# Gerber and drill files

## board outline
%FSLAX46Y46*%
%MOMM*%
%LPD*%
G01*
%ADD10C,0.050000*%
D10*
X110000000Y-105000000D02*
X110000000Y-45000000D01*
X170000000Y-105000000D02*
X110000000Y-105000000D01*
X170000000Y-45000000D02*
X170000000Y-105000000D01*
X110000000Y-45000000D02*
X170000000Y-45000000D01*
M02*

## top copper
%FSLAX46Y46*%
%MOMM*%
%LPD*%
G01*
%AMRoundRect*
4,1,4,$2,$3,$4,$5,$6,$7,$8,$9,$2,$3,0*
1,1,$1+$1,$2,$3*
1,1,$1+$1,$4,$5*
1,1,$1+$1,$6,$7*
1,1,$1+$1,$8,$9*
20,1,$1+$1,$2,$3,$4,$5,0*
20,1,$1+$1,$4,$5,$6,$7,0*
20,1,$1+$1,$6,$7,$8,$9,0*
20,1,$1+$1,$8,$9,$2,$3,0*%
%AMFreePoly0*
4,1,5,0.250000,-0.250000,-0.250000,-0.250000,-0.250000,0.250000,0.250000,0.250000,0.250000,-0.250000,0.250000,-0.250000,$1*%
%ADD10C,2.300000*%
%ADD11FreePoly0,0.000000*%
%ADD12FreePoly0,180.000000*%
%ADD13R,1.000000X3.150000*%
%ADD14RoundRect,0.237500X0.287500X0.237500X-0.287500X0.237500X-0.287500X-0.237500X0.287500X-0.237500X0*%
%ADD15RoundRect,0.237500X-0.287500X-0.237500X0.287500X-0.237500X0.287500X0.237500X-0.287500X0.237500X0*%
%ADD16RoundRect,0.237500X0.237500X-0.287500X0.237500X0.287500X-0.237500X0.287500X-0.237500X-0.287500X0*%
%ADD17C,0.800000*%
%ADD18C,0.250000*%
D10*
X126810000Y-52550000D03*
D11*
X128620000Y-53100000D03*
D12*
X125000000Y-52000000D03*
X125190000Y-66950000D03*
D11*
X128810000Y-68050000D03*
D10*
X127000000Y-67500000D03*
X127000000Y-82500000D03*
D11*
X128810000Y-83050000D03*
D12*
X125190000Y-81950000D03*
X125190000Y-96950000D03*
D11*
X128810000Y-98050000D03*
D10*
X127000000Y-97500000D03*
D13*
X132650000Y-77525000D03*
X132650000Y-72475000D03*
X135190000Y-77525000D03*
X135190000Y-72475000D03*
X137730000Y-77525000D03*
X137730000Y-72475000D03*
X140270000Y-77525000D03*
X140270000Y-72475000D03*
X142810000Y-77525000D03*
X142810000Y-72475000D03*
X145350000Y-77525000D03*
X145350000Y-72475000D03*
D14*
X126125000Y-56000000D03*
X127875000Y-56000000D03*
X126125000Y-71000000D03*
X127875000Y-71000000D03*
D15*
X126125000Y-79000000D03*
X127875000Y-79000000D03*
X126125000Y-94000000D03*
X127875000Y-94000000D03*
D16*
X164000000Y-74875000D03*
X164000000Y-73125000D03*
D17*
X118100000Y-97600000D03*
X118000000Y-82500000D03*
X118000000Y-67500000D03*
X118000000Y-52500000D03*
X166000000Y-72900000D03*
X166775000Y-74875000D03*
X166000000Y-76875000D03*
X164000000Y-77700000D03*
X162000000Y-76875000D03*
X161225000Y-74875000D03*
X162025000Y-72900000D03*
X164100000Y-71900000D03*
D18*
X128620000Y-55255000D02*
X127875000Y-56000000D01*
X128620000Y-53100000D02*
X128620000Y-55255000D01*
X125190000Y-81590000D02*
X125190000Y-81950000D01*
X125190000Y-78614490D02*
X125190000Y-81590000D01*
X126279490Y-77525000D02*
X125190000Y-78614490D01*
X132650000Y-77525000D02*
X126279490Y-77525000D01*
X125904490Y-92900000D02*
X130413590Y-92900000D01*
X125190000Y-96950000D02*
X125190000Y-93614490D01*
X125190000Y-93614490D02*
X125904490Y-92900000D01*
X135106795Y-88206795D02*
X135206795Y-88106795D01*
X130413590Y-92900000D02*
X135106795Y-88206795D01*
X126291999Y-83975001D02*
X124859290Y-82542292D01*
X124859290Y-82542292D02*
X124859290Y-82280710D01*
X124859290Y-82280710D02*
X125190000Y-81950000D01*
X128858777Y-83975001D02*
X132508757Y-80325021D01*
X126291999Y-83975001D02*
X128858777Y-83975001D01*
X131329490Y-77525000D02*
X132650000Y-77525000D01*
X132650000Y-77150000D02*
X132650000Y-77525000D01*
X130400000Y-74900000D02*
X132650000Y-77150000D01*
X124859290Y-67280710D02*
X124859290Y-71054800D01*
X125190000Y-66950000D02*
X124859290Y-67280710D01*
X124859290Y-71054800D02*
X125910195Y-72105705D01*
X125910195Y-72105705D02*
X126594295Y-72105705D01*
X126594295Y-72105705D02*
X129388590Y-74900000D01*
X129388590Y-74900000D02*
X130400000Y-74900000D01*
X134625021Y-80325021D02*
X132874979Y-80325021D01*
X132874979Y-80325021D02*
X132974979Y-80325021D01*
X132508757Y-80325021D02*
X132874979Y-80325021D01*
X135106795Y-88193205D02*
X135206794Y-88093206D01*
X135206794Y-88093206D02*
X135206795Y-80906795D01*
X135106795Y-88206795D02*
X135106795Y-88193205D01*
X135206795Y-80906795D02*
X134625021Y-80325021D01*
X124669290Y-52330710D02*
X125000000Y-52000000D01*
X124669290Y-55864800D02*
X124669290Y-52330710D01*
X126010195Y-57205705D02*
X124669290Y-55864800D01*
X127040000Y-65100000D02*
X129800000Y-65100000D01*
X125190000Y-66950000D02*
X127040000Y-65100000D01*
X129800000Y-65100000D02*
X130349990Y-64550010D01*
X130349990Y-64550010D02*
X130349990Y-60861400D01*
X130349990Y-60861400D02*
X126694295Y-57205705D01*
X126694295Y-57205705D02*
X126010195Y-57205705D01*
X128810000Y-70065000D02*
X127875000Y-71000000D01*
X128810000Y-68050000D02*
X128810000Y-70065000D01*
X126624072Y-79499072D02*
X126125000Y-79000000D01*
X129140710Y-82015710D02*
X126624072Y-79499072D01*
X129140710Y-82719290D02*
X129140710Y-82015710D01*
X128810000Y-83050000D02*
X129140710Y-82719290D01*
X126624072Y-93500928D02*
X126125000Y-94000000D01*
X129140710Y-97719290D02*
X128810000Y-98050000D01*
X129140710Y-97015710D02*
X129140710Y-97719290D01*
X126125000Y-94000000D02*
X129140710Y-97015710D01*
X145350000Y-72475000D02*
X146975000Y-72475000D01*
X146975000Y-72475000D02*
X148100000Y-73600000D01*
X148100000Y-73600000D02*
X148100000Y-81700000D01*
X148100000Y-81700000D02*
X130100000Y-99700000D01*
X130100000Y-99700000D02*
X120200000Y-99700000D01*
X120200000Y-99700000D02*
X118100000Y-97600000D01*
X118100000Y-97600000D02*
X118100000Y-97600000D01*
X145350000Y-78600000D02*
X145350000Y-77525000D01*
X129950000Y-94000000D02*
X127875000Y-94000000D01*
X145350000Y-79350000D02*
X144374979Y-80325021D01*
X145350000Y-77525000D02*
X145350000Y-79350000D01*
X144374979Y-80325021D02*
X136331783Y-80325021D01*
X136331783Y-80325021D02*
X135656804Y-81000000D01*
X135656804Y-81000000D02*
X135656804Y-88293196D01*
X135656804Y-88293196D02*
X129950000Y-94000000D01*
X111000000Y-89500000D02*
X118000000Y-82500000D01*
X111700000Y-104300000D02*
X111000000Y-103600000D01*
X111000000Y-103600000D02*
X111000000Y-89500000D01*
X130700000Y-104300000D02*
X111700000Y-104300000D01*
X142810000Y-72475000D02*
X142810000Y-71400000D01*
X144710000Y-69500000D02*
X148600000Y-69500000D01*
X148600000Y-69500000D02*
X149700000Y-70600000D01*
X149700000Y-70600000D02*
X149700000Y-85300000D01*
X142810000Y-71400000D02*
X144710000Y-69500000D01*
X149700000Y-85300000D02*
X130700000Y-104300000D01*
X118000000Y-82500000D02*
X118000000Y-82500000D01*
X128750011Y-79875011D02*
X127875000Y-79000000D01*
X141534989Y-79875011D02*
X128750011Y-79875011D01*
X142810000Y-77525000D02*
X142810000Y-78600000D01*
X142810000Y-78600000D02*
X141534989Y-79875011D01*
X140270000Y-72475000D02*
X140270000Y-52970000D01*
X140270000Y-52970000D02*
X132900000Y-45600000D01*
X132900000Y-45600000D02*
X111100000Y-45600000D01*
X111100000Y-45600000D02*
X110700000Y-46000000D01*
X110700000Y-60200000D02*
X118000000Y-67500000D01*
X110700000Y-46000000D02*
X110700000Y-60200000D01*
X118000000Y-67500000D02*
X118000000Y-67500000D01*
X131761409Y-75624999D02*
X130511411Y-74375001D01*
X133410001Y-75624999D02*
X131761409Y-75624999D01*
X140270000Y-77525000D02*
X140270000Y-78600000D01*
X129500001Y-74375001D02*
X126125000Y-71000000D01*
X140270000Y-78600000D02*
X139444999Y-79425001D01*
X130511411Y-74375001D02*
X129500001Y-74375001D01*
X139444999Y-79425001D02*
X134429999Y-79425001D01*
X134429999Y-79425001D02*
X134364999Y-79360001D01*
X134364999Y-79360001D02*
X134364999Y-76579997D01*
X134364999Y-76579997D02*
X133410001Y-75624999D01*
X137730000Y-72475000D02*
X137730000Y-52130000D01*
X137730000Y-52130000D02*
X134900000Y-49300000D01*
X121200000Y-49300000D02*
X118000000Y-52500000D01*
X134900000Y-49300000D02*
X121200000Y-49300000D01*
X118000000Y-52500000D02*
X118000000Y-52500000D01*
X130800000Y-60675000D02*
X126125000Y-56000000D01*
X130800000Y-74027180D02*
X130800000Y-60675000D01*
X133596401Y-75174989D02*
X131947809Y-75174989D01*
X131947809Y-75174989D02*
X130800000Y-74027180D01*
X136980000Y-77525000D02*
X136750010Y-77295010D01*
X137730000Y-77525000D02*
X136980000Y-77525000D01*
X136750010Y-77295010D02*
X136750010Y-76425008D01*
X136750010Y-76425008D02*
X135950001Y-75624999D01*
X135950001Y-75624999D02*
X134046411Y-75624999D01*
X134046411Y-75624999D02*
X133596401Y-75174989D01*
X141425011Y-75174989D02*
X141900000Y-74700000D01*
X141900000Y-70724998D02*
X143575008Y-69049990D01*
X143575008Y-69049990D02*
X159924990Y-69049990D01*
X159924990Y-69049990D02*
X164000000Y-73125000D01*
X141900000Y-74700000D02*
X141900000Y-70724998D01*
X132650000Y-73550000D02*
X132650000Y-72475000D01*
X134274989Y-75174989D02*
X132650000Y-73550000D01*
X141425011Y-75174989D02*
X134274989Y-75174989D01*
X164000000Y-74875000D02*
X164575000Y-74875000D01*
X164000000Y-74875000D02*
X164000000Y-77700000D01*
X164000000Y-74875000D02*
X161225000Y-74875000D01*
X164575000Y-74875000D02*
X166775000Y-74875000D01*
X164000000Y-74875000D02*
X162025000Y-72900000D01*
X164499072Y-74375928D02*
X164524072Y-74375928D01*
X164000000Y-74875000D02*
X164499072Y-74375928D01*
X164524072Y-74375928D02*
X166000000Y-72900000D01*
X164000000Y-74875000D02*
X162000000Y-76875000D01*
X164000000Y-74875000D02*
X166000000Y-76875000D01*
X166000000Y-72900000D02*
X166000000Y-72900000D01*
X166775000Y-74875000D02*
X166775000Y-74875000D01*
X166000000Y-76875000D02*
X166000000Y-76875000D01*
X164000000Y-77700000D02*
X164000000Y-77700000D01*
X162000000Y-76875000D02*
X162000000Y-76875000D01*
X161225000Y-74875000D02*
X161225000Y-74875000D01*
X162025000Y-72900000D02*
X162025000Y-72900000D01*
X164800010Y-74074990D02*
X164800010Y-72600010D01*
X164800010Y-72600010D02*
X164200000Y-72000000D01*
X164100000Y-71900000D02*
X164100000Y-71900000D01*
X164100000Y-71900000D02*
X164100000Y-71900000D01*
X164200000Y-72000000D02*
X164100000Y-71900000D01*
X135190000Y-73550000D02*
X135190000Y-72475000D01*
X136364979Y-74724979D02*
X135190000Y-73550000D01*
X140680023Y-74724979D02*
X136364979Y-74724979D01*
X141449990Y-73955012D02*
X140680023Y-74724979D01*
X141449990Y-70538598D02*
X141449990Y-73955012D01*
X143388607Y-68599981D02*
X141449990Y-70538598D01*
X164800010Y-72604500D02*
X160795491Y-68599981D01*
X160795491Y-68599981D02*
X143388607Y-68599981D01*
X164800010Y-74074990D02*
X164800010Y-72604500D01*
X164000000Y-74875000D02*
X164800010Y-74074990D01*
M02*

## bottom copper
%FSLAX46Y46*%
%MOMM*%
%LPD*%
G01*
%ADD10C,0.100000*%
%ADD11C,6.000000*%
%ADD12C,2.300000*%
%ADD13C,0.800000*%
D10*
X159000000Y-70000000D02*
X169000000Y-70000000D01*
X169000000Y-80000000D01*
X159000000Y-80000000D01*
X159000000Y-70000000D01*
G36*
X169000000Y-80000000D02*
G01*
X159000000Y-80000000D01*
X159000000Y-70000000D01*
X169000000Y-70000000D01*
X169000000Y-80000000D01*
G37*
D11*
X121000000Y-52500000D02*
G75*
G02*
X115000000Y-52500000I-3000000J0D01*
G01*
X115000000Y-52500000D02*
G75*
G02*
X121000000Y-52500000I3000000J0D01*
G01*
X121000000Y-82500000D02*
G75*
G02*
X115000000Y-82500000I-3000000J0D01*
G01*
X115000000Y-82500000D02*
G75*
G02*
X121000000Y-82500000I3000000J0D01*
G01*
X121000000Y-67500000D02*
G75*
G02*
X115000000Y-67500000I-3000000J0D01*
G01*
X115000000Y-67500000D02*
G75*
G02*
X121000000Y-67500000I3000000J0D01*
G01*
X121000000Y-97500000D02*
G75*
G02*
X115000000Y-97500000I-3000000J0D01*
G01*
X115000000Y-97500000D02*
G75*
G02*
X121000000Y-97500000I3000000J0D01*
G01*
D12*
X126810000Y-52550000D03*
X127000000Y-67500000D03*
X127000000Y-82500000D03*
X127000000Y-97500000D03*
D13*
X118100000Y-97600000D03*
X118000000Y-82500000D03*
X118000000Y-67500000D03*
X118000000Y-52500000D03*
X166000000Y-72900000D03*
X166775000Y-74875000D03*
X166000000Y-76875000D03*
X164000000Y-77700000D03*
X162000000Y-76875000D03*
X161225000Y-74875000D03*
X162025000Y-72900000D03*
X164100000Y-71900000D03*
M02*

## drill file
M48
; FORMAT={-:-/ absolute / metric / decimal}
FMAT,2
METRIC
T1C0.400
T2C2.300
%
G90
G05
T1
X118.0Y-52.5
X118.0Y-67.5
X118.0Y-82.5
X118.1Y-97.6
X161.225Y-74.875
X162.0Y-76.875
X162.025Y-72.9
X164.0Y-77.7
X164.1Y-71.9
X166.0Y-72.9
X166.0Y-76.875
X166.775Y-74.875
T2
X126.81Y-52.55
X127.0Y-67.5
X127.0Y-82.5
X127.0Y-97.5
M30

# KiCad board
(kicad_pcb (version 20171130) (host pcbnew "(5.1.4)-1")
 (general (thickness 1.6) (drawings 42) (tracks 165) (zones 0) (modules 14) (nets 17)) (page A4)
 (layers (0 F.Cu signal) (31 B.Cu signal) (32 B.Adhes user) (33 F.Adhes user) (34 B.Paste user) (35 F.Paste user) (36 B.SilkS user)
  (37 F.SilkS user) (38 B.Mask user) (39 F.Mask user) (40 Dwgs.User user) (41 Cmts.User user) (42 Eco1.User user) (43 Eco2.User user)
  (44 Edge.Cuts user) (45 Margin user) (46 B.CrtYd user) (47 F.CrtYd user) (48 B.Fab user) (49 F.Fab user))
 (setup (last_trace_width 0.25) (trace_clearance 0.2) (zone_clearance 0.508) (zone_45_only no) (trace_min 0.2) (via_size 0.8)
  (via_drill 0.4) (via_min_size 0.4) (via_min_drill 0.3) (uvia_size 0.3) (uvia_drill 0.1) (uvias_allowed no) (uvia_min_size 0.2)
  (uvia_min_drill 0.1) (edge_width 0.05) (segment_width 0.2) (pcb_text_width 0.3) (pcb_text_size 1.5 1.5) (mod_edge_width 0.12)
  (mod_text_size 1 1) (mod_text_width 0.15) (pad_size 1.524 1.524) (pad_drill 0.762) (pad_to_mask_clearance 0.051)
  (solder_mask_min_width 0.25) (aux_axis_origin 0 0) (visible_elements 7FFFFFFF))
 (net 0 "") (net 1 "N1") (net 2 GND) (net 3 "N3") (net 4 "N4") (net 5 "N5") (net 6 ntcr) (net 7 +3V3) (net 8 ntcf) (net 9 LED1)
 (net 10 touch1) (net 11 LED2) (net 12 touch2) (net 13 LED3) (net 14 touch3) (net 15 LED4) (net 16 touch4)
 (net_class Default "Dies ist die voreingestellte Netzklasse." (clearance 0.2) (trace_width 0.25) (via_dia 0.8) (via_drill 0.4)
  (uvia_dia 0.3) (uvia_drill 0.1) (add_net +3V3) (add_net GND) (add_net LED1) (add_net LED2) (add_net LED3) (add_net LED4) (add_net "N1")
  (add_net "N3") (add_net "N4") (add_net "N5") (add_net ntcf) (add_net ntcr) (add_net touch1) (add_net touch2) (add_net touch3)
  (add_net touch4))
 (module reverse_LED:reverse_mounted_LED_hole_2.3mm (layer F.Cu) (at 126.81 52.55)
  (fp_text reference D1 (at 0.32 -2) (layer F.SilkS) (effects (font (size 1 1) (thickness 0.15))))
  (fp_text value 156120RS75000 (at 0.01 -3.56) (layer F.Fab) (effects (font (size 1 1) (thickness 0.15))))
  (pad 0 thru_hole circle (at 0 0) (size 2.3 2.3) (drill 2.3) (layers *.Cu *.Mask))
  (pad 2 smd custom (at 1.81 0.55) (size 0.5 0.5) (layers F.Cu F.Paste F.Mask) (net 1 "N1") (zone_connect 0)
   (options (clearance outline) (anchor rect)) (primitives))
  (pad 1 smd custom (at -1.81 -0.55 180) (size 0.5 0.5) (layers F.Cu F.Paste F.Mask) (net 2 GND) (zone_connect 0)
   (options (clearance outline) (anchor rect)) (primitives)))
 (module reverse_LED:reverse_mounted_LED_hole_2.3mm (layer F.Cu) (at 127 67.5)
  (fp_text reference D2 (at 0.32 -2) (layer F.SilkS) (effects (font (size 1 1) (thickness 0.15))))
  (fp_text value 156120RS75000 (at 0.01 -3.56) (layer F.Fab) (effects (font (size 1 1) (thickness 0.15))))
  (pad 1 smd custom (at -1.81 -0.55 180) (size 0.5 0.5) (layers F.Cu F.Paste F.Mask) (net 2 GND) (zone_connect 0)
   (options (clearance outline) (anchor rect)) (primitives))
  (pad 2 smd custom (at 1.81 0.55) (size 0.5 0.5) (layers F.Cu F.Paste F.Mask) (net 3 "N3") (zone_connect 0)
   (options (clearance outline) (anchor rect)) (primitives))
  (pad 0 thru_hole circle (at 0 0) (size 2.3 2.3) (drill 2.3) (layers *.Cu *.Mask)))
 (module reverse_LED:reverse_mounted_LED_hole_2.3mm (layer F.Cu) (at 127 82.5)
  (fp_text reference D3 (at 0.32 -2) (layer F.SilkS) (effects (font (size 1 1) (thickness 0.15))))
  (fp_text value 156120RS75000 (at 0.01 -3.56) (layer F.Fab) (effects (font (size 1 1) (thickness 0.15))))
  (pad 0 thru_hole circle (at 0 0) (size 2.3 2.3) (drill 2.3) (layers *.Cu *.Mask))
  (pad 2 smd custom (at 1.81 0.55) (size 0.5 0.5) (layers F.Cu F.Paste F.Mask) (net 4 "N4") (zone_connect 0)
   (options (clearance outline) (anchor rect)) (primitives))
  (pad 1 smd custom (at -1.81 -0.55 180) (size 0.5 0.5) (layers F.Cu F.Paste F.Mask) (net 2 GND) (zone_connect 0)
   (options (clearance outline) (anchor rect)) (primitives)))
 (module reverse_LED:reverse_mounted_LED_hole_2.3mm (layer F.Cu) (at 127 97.5)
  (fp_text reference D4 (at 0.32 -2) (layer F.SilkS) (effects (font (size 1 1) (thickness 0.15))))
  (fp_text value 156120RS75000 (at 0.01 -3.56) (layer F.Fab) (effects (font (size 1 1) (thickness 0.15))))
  (pad 1 smd custom (at -1.81 -0.55 180) (size 0.5 0.5) (layers F.Cu F.Paste F.Mask) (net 2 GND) (zone_connect 0)
   (options (clearance outline) (anchor rect)) (primitives))
  (pad 2 smd custom (at 1.81 0.55) (size 0.5 0.5) (layers F.Cu F.Paste F.Mask) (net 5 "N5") (zone_connect 0)
   (options (clearance outline) (anchor rect)) (primitives))
  (pad 0 thru_hole circle (at 0 0) (size 2.3 2.3) (drill 2.3) (layers *.Cu *.Mask)))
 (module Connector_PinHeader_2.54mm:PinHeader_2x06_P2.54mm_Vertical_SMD (layer F.Cu) (at 139 75 90)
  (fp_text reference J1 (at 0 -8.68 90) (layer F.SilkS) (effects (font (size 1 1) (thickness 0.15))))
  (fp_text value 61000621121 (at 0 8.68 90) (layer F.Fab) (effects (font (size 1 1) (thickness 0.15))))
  (pad 1 smd rect (at -2.525 -6.35 90) (size 3.15 1) (layers F.Cu F.Paste F.Mask) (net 2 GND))
  (pad 2 smd rect (at 2.525 -6.35 90) (size 3.15 1) (layers F.Cu F.Paste F.Mask) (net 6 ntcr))
  (pad 3 smd rect (at -2.525 -3.81 90) (size 3.15 1) (layers F.Cu F.Paste F.Mask) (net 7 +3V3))
  (pad 4 smd rect (at 2.525 -3.81 90) (size 3.15 1) (layers F.Cu F.Paste F.Mask) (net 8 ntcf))
  (pad 5 smd rect (at -2.525 -1.27 90) (size 3.15 1) (layers F.Cu F.Paste F.Mask) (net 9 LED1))
  (pad 6 smd rect (at 2.525 -1.27 90) (size 3.15 1) (layers F.Cu F.Paste F.Mask) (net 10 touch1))
  (pad 7 smd rect (at -2.525 1.27 90) (size 3.15 1) (layers F.Cu F.Paste F.Mask) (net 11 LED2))
  (pad 8 smd rect (at 2.525 1.27 90) (size 3.15 1) (layers F.Cu F.Paste F.Mask) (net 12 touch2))
  (pad 9 smd rect (at -2.525 3.81 90) (size 3.15 1) (layers F.Cu F.Paste F.Mask) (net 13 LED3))
  (pad 10 smd rect (at 2.525 3.81 90) (size 3.15 1) (layers F.Cu F.Paste F.Mask) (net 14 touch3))
  (pad 11 smd rect (at -2.525 6.35 90) (size 3.15 1) (layers F.Cu F.Paste F.Mask) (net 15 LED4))
  (pad 12 smd rect (at 2.525 6.35 90) (size 3.15 1) (layers F.Cu F.Paste F.Mask) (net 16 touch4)))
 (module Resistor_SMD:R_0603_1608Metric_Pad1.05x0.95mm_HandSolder (layer F.Cu) (at 127 56 180)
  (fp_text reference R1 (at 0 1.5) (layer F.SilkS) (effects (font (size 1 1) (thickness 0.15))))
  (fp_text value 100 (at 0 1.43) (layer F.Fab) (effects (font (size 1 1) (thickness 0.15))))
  (pad 2 smd roundrect (at 0.875 0 180) (size 1.05 0.95) (layers F.Cu F.Paste F.Mask) (roundrect_rratio 0.25) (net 9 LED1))
  (pad 1 smd roundrect (at -0.875 0 180) (size 1.05 0.95) (layers F.Cu F.Paste F.Mask) (roundrect_rratio 0.25) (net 1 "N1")))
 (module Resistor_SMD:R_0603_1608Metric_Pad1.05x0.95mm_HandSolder (layer F.Cu) (at 127 71 180)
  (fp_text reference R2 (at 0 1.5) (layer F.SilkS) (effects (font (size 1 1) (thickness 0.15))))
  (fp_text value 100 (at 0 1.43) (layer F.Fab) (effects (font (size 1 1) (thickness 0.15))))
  (pad 2 smd roundrect (at 0.875 0 180) (size 1.05 0.95) (layers F.Cu F.Paste F.Mask) (roundrect_rratio 0.25) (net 11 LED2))
  (pad 1 smd roundrect (at -0.875 0 180) (size 1.05 0.95) (layers F.Cu F.Paste F.Mask) (roundrect_rratio 0.25) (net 3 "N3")))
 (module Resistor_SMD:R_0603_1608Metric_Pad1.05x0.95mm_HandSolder (layer F.Cu) (at 127 79)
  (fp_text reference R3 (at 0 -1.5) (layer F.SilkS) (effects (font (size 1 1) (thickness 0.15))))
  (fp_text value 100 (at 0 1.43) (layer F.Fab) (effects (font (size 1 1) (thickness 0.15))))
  (pad 1 smd roundrect (at -0.875 0) (size 1.05 0.95) (layers F.Cu F.Paste F.Mask) (roundrect_rratio 0.25) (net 4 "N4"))
  (pad 2 smd roundrect (at 0.875 0) (size 1.05 0.95) (layers F.Cu F.Paste F.Mask) (roundrect_rratio 0.25) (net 13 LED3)))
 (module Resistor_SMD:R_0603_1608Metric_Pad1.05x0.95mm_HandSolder (layer F.Cu) (at 127 94)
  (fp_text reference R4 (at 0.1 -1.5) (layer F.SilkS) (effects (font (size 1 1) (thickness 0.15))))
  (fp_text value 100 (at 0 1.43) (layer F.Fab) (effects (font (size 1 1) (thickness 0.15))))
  (pad 1 smd roundrect (at -0.875 0) (size 1.05 0.95) (layers F.Cu F.Paste F.Mask) (roundrect_rratio 0.25) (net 5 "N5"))
  (pad 2 smd roundrect (at 0.875 0) (size 1.05 0.95) (layers F.Cu F.Paste F.Mask) (roundrect_rratio 0.25) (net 15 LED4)))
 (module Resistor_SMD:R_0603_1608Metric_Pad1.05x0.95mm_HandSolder (layer F.Cu) (at 164 74 90)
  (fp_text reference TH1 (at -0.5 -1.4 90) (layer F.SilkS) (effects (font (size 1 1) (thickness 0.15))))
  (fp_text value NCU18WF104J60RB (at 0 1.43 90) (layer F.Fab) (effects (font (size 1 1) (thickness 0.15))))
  (pad 1 smd roundrect (at -0.875 0 90) (size 1.05 0.95) (layers F.Cu F.Paste F.Mask) (roundrect_rratio 0.25) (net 8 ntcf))
  (pad 2 smd roundrect (at 0.875 0 90) (size 1.05 0.95) (layers F.Cu F.Paste F.Mask) (roundrect_rratio 0.25) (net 6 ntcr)))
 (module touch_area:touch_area (layer F.Cu) (at 118 52.5)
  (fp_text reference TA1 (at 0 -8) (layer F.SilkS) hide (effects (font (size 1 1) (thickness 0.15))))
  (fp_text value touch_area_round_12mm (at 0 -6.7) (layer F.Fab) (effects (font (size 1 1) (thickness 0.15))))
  (fp_circle (center 0 0) (end 3 0) (layer B.Cu) (width 6)))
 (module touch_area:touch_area (layer F.Cu) (at 118 82.5)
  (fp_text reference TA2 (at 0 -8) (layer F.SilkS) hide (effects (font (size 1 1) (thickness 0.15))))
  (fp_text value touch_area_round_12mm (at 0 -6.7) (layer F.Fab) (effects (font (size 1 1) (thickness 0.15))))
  (fp_circle (center 0 0) (end 3 0) (layer B.Cu) (width 6)))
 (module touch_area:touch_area (layer F.Cu) (at 118 67.5)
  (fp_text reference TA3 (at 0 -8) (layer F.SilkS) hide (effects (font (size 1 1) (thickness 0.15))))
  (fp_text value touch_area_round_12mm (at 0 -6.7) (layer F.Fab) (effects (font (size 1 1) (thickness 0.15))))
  (fp_circle (center 0 0) (end 3 0) (layer B.Cu) (width 6)))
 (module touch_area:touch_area (layer F.Cu) (at 118 97.5)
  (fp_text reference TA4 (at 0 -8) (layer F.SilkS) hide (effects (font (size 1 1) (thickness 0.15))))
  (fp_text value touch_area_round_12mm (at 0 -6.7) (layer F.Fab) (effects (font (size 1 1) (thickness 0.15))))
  (fp_circle (center 0 0) (end 3 0) (layer B.Cu) (width 6)))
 (gr_poly (pts (xy 159 70) (xy 169 70) (xy 169 80) (xy 159 80)) (layer B.Cu) (width 0.1))
 (gr_line (start 110 105) (end 110 45) (layer Edge.Cuts) (width 0.05))
 (gr_line (start 170 105) (end 110 105) (layer Edge.Cuts) (width 0.05))
 (gr_line (start 170 45) (end 170 105) (layer Edge.Cuts) (width 0.05))
 (gr_line (start 110 45) (end 170 45) (layer Edge.Cuts) (width 0.05))
 (segment (start 128.62 55.255) (end 127.875 56) (width 0.25) (layer F.Cu) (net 1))
 (segment (start 128.62 53.1) (end 128.62 55.255) (width 0.25) (layer F.Cu) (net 1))
 (segment (start 125.19 81.59) (end 125.19 81.95) (width 0.25) (layer F.Cu) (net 2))
 (segment (start 125.19 78.61449) (end 125.19 81.59) (width 0.25) (layer F.Cu) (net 2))
 (segment (start 126.27949 77.525) (end 125.19 78.61449) (width 0.25) (layer F.Cu) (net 2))
 (segment (start 132.65 77.525) (end 126.27949 77.525) (width 0.25) (layer F.Cu) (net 2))
 (segment (start 125.90449 92.9) (end 130.41359 92.9) (width 0.25) (layer F.Cu) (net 2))
 (segment (start 125.19 96.95) (end 125.19 93.61449) (width 0.25) (layer F.Cu) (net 2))
 (segment (start 125.19 93.61449) (end 125.90449 92.9) (width 0.25) (layer F.Cu) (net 2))
 (segment (start 135.106795 88.206795) (end 135.206795 88.106795) (width 0.25) (layer F.Cu) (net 2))
 (segment (start 130.41359 92.9) (end 135.106795 88.206795) (width 0.25) (layer F.Cu) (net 2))
 (segment (start 126.291999 83.975001) (end 124.85929 82.542292) (width 0.25) (layer F.Cu) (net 2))
 (segment (start 124.85929 82.542292) (end 124.85929 82.28071) (width 0.25) (layer F.Cu) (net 2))
 (segment (start 124.85929 82.28071) (end 125.19 81.95) (width 0.25) (layer F.Cu) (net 2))
 (segment (start 128.858777 83.975001) (end 132.508757 80.325021) (width 0.25) (layer F.Cu) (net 2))
 (segment (start 126.291999 83.975001) (end 128.858777 83.975001) (width 0.25) (layer F.Cu) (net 2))
 (segment (start 131.32949 77.525) (end 132.65 77.525) (width 0.25) (layer F.Cu) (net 2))
 (segment (start 132.65 77.15) (end 132.65 77.525) (width 0.25) (layer F.Cu) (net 2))
 (segment (start 130.4 74.9) (end 132.65 77.15) (width 0.25) (layer F.Cu) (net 2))
 (segment (start 124.85929 67.28071) (end 124.85929 71.0548) (width 0.25) (layer F.Cu) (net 2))
 (segment (start 125.19 66.95) (end 124.85929 67.28071) (width 0.25) (layer F.Cu) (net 2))
 (segment (start 124.85929 71.0548) (end 125.910195 72.105705) (width 0.25) (layer F.Cu) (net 2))
 (segment (start 125.910195 72.105705) (end 126.594295 72.105705) (width 0.25) (layer F.Cu) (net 2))
 (segment (start 126.594295 72.105705) (end 129.38859 74.9) (width 0.25) (layer F.Cu) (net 2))
 (segment (start 129.38859 74.9) (end 130.4 74.9) (width 0.25) (layer F.Cu) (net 2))
 (segment (start 134.625021 80.325021) (end 132.874979 80.325021) (width 0.25) (layer F.Cu) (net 2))
 (segment (start 132.874979 80.325021) (end 132.974979 80.325021) (width 0.25) (layer F.Cu) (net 2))
 (segment (start 132.508757 80.325021) (end 132.874979 80.325021) (width 0.25) (layer F.Cu) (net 2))
 (segment (start 135.106795 88.193205) (end 135.206794 88.093206) (width 0.25) (layer F.Cu) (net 2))
 (segment (start 135.206794 88.093206) (end 135.206795 80.906795) (width 0.25) (layer F.Cu) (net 2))
 (segment (start 135.106795 88.206795) (end 135.106795 88.193205) (width 0.25) (layer F.Cu) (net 2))
 (segment (start 135.206795 80.906795) (end 134.625021 80.325021) (width 0.25) (layer F.Cu) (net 2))
 (segment (start 124.66929 52.33071) (end 125 52) (width 0.25) (layer F.Cu) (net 2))
 (segment (start 124.66929 55.8648) (end 124.66929 52.33071) (width 0.25) (layer F.Cu) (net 2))
 (segment (start 126.010195 57.205705) (end 124.66929 55.8648) (width 0.25) (layer F.Cu) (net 2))
 (segment (start 127.04 65.1) (end 129.8 65.1) (width 0.25) (layer F.Cu) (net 2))
 (segment (start 125.19 66.95) (end 127.04 65.1) (width 0.25) (layer F.Cu) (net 2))
 (segment (start 129.8 65.1) (end 130.34999 64.55001) (width 0.25) (layer F.Cu) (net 2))
 (segment (start 130.34999 64.55001) (end 130.34999 60.8614) (width 0.25) (layer F.Cu) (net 2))
 (segment (start 130.34999 60.8614) (end 126.694295 57.205705) (width 0.25) (layer F.Cu) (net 2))
 (segment (start 126.694295 57.205705) (end 126.010195 57.205705) (width 0.25) (layer F.Cu) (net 2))
 (segment (start 128.81 70.065) (end 127.875 71) (width 0.25) (layer F.Cu) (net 3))
 (segment (start 128.81 68.05) (end 128.81 70.065) (width 0.25) (layer F.Cu) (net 3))
 (segment (start 126.624072 79.499072) (end 126.125 79) (width 0.25) (layer F.Cu) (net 4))
 (segment (start 129.14071 82.01571) (end 126.624072 79.499072) (width 0.25) (layer F.Cu) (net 4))
 (segment (start 129.14071 82.71929) (end 129.14071 82.01571) (width 0.25) (layer F.Cu) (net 4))
 (segment (start 128.81 83.05) (end 129.14071 82.71929) (width 0.25) (layer F.Cu) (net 4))
 (segment (start 126.624072 93.500928) (end 126.125 94) (width 0.25) (layer F.Cu) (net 5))
 (segment (start 129.14071 97.71929) (end 128.81 98.05) (width 0.25) (layer F.Cu) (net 5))
 (segment (start 129.14071 97.01571) (end 129.14071 97.71929) (width 0.25) (layer F.Cu) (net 5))
 (segment (start 126.125 94) (end 129.14071 97.01571) (width 0.25) (layer F.Cu) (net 5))
 (segment (start 145.35 72.475) (end 146.975 72.475) (width 0.25) (layer F.Cu) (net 16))
 (segment (start 146.975 72.475) (end 148.1 73.6) (width 0.25) (layer F.Cu) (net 16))
 (segment (start 148.1 73.6) (end 148.1 81.7) (width 0.25) (layer F.Cu) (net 16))
 (segment (start 148.1 81.7) (end 130.1 99.7) (width 0.25) (layer F.Cu) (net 16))
 (segment (start 130.1 99.7) (end 120.2 99.7) (width 0.25) (layer F.Cu) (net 16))
 (segment (start 120.2 99.7) (end 118.1 97.6) (width 0.25) (layer F.Cu) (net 16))
 (segment (start 118.1 97.6) (end 118.1 97.6) (width 0.25) (layer F.Cu) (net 16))
 (via (at 118.1 97.6) (size 0.8) (drill 0.4) (layers F.Cu B.Cu) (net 16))
 (segment (start 145.35 78.6) (end 145.35 77.525) (width 0.25) (layer F.Cu) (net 15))
 (segment (start 129.95 94) (end 127.875 94) (width 0.25) (layer F.Cu) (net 15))
 (segment (start 145.35 79.35) (end 144.374979 80.325021) (width 0.25) (layer F.Cu) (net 15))
 (segment (start 145.35 77.525) (end 145.35 79.35) (width 0.25) (layer F.Cu) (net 15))
 (segment (start 144.374979 80.325021) (end 136.331783 80.325021) (width 0.25) (layer F.Cu) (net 15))
 (segment (start 136.331783 80.325021) (end 135.656804 81) (width 0.25) (layer F.Cu) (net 15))
 (segment (start 135.656804 81) (end 135.656804 88.293196) (width 0.25) (layer F.Cu) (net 15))
 (segment (start 135.656804 88.293196) (end 129.95 94) (width 0.25) (layer F.Cu) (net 15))
 (segment (start 111 89.5) (end 118 82.5) (width 0.25) (layer F.Cu) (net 14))
 (segment (start 111.7 104.3) (end 111 103.6) (width 0.25) (layer F.Cu) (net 14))
 (segment (start 111 103.6) (end 111 89.5) (width 0.25) (layer F.Cu) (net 14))
 (segment (start 130.7 104.3) (end 111.7 104.3) (width 0.25) (layer F.Cu) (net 14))
 (segment (start 142.81 72.475) (end 142.81 71.4) (width 0.25) (layer F.Cu) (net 14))
 (segment (start 144.71 69.5) (end 148.6 69.5) (width 0.25) (layer F.Cu) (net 14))
 (segment (start 148.6 69.5) (end 149.7 70.6) (width 0.25) (layer F.Cu) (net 14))
 (segment (start 149.7 70.6) (end 149.7 85.3) (width 0.25) (layer F.Cu) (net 14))
 (segment (start 142.81 71.4) (end 144.71 69.5) (width 0.25) (layer F.Cu) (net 14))
 (segment (start 149.7 85.3) (end 130.7 104.3) (width 0.25) (layer F.Cu) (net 14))
 (segment (start 118 82.5) (end 118 82.5) (width 0.25) (layer F.Cu) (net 14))
 (via (at 118 82.5) (size 0.8) (drill 0.4) (layers F.Cu B.Cu) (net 14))
 (segment (start 128.750011 79.875011) (end 127.875 79) (width 0.25) (layer F.Cu) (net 13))
 (segment (start 141.534989 79.875011) (end 128.750011 79.875011) (width 0.25) (layer F.Cu) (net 13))
 (segment (start 142.81 77.525) (end 142.81 78.6) (width 0.25) (layer F.Cu) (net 13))
 (segment (start 142.81 78.6) (end 141.534989 79.875011) (width 0.25) (layer F.Cu) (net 13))
 (segment (start 140.27 72.475) (end 140.27 52.97) (width 0.25) (layer F.Cu) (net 12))
 (segment (start 140.27 52.97) (end 132.9 45.6) (width 0.25) (layer F.Cu) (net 12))
 (segment (start 132.9 45.6) (end 111.1 45.6) (width 0.25) (layer F.Cu) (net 12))
 (segment (start 111.1 45.6) (end 110.7 46) (width 0.25) (layer F.Cu) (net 12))
 (segment (start 110.7 60.2) (end 118 67.5) (width 0.25) (layer F.Cu) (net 12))
 (segment (start 110.7 46) (end 110.7 60.2) (width 0.25) (layer F.Cu) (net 12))
 (segment (start 118 67.5) (end 118 67.5) (width 0.25) (layer F.Cu) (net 12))
 (via (at 118 67.5) (size 0.8) (drill 0.4) (layers F.Cu B.Cu) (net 12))
 (segment (start 131.761409 75.624999) (end 130.511411 74.375001) (width 0.25) (layer F.Cu) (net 11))
 (segment (start 133.410001 75.624999) (end 131.761409 75.624999) (width 0.25) (layer F.Cu) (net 11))
 (segment (start 140.27 77.525) (end 140.27 78.6) (width 0.25) (layer F.Cu) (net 11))
 (segment (start 129.500001 74.375001) (end 126.125 71) (width 0.25) (layer F.Cu) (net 11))
 (segment (start 140.27 78.6) (end 139.444999 79.425001) (width 0.25) (layer F.Cu) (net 11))
 (segment (start 130.511411 74.375001) (end 129.500001 74.375001) (width 0.25) (layer F.Cu) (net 11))
 (segment (start 139.444999 79.425001) (end 134.429999 79.425001) (width 0.25) (layer F.Cu) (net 11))
 (segment (start 134.429999 79.425001) (end 134.364999 79.360001) (width 0.25) (layer F.Cu) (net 11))
 (segment (start 134.364999 79.360001) (end 134.364999 76.579997) (width 0.25) (layer F.Cu) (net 11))
 (segment (start 134.364999 76.579997) (end 133.410001 75.624999) (width 0.25) (layer F.Cu) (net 11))
 (segment (start 137.73 72.475) (end 137.73 52.13) (width 0.25) (layer F.Cu) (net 10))
 (segment (start 137.73 52.13) (end 134.9 49.3) (width 0.25) (layer F.Cu) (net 10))
 (segment (start 121.2 49.3) (end 118 52.5) (width 0.25) (layer F.Cu) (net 10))
 (segment (start 134.9 49.3) (end 121.2 49.3) (width 0.25) (layer F.Cu) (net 10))
 (segment (start 118 52.5) (end 118 52.5) (width 0.25) (layer F.Cu) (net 10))
 (via (at 118 52.5) (size 0.8) (drill 0.4) (layers F.Cu B.Cu) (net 10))
 (segment (start 130.8 60.675) (end 126.125 56) (width 0.25) (layer F.Cu) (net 9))
 (segment (start 130.8 74.02718) (end 130.8 60.675) (width 0.25) (layer F.Cu) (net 9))
 (segment (start 133.596401 75.174989) (end 131.947809 75.174989) (width 0.25) (layer F.Cu) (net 9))
 (segment (start 131.947809 75.174989) (end 130.8 74.02718) (width 0.25) (layer F.Cu) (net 9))
 (segment (start 136.98 77.525) (end 136.75001 77.29501) (width 0.25) (layer F.Cu) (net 9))
 (segment (start 137.73 77.525) (end 136.98 77.525) (width 0.25) (layer F.Cu) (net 9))
 (segment (start 136.75001 77.29501) (end 136.75001 76.425008) (width 0.25) (layer F.Cu) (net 9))
 (segment (start 136.75001 76.425008) (end 135.950001 75.624999) (width 0.25) (layer F.Cu) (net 9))
 (segment (start 135.950001 75.624999) (end 134.046411 75.624999) (width 0.25) (layer F.Cu) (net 9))
 (segment (start 134.046411 75.624999) (end 133.596401 75.174989) (width 0.25) (layer F.Cu) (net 9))
 (segment (start 141.425011 75.174989) (end 141.9 74.7) (width 0.25) (layer F.Cu) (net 6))
 (segment (start 141.9 70.724998) (end 143.575008 69.04999) (width 0.25) (layer F.Cu) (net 6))
 (segment (start 143.575008 69.04999) (end 159.92499 69.04999) (width 0.25) (layer F.Cu) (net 6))
 (segment (start 159.92499 69.04999) (end 164 73.125) (width 0.25) (layer F.Cu) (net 6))
 (segment (start 141.9 74.7) (end 141.9 70.724998) (width 0.25) (layer F.Cu) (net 6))
 (segment (start 132.65 73.55) (end 132.65 72.475) (width 0.25) (layer F.Cu) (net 6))
 (segment (start 134.274989 75.174989) (end 132.65 73.55) (width 0.25) (layer F.Cu) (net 6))
 (segment (start 141.425011 75.174989) (end 134.274989 75.174989) (width 0.25) (layer F.Cu) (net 6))
 (segment (start 164 74.875) (end 164.575 74.875) (width 0.25) (layer F.Cu) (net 8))
 (segment (start 164 74.875) (end 164 77.7) (width 0.25) (layer F.Cu) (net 8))
 (segment (start 164 74.875) (end 161.225 74.875) (width 0.25) (layer F.Cu) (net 8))
 (segment (start 164.575 74.875) (end 166.775 74.875) (width 0.25) (layer F.Cu) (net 8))
 (segment (start 164 74.875) (end 162.025 72.9) (width 0.25) (layer F.Cu) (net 8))
 (segment (start 164.499072 74.375928) (end 164.524072 74.375928) (width 0.25) (layer F.Cu) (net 8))
 (segment (start 164 74.875) (end 164.499072 74.375928) (width 0.25) (layer F.Cu) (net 8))
 (segment (start 164.524072 74.375928) (end 166 72.9) (width 0.25) (layer F.Cu) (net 8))
 (segment (start 164 74.875) (end 162 76.875) (width 0.25) (layer F.Cu) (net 8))
 (segment (start 164 74.875) (end 166 76.875) (width 0.25) (layer F.Cu) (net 8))
 (segment (start 166 72.9) (end 166 72.9) (width 0.25) (layer F.Cu) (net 8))
 (via (at 166 72.9) (size 0.8) (drill 0.4) (layers F.Cu B.Cu) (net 8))
 (segment (start 166.775 74.875) (end 166.775 74.875) (width 0.25) (layer F.Cu) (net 8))
 (via (at 166.775 74.875) (size 0.8) (drill 0.4) (layers F.Cu B.Cu) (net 8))
 (segment (start 166 76.875) (end 166 76.875) (width 0.25) (layer F.Cu) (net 8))
 (via (at 166 76.875) (size 0.8) (drill 0.4) (layers F.Cu B.Cu) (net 8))
 (segment (start 164 77.7) (end 164 77.7) (width 0.25) (layer F.Cu) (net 8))
 (via (at 164 77.7) (size 0.8) (drill 0.4) (layers F.Cu B.Cu) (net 8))
 (segment (start 162 76.875) (end 162 76.875) (width 0.25) (layer F.Cu) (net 8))
 (via (at 162 76.875) (size 0.8) (drill 0.4) (layers F.Cu B.Cu) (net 8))
 (segment (start 161.225 74.875) (end 161.225 74.875) (width 0.25) (layer F.Cu) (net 8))
 (via (at 161.225 74.875) (size 0.8) (drill 0.4) (layers F.Cu B.Cu) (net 8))
 (segment (start 162.025 72.9) (end 162.025 72.9) (width 0.25) (layer F.Cu) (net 8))
 (via (at 162.025 72.9) (size 0.8) (drill 0.4) (layers F.Cu B.Cu) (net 8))
 (segment (start 164.80001 74.07499) (end 164.80001 72.60001) (width 0.25) (layer F.Cu) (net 8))
 (segment (start 164.80001 72.60001) (end 164.2 72) (width 0.25) (layer F.Cu) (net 8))
 (segment (start 164.1 71.9) (end 164.1 71.9) (width 0.25) (layer F.Cu) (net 8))
 (segment (start 164.1 71.9) (end 164.1 71.9) (width 0.25) (layer F.Cu) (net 8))
 (segment (start 164.2 72) (end 164.1 71.9) (width 0.25) (layer F.Cu) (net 8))
 (via (at 164.1 71.9) (size 0.8) (drill 0.4) (layers F.Cu B.Cu) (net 8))
 (segment (start 135.19 73.55) (end 135.19 72.475) (width 0.25) (layer F.Cu) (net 8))
 (segment (start 136.364979 74.724979) (end 135.19 73.55) (width 0.25) (layer F.Cu) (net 8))
 (segment (start 140.680023 74.724979) (end 136.364979 74.724979) (width 0.25) (layer F.Cu) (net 8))
 (segment (start 141.44999 73.955012) (end 140.680023 74.724979) (width 0.25) (layer F.Cu) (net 8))
 (segment (start 141.44999 70.538598) (end 141.44999 73.955012) (width 0.25) (layer F.Cu) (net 8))
 (segment (start 143.388607 68.599981) (end 141.44999 70.538598) (width 0.25) (layer F.Cu) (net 8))
 (segment (start 164.80001 72.6045) (end 160.795491 68.599981) (width 0.25) (layer F.Cu) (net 8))
 (segment (start 160.795491 68.599981) (end 143.388607 68.599981) (width 0.25) (layer F.Cu) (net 8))
 (segment (start 164.80001 74.07499) (end 164.80001 72.6045) (width 0.25) (layer F.Cu) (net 8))
 (segment (start 164 74.875) (end 164.80001 74.07499) (width 0.25) (layer F.Cu) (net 8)))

